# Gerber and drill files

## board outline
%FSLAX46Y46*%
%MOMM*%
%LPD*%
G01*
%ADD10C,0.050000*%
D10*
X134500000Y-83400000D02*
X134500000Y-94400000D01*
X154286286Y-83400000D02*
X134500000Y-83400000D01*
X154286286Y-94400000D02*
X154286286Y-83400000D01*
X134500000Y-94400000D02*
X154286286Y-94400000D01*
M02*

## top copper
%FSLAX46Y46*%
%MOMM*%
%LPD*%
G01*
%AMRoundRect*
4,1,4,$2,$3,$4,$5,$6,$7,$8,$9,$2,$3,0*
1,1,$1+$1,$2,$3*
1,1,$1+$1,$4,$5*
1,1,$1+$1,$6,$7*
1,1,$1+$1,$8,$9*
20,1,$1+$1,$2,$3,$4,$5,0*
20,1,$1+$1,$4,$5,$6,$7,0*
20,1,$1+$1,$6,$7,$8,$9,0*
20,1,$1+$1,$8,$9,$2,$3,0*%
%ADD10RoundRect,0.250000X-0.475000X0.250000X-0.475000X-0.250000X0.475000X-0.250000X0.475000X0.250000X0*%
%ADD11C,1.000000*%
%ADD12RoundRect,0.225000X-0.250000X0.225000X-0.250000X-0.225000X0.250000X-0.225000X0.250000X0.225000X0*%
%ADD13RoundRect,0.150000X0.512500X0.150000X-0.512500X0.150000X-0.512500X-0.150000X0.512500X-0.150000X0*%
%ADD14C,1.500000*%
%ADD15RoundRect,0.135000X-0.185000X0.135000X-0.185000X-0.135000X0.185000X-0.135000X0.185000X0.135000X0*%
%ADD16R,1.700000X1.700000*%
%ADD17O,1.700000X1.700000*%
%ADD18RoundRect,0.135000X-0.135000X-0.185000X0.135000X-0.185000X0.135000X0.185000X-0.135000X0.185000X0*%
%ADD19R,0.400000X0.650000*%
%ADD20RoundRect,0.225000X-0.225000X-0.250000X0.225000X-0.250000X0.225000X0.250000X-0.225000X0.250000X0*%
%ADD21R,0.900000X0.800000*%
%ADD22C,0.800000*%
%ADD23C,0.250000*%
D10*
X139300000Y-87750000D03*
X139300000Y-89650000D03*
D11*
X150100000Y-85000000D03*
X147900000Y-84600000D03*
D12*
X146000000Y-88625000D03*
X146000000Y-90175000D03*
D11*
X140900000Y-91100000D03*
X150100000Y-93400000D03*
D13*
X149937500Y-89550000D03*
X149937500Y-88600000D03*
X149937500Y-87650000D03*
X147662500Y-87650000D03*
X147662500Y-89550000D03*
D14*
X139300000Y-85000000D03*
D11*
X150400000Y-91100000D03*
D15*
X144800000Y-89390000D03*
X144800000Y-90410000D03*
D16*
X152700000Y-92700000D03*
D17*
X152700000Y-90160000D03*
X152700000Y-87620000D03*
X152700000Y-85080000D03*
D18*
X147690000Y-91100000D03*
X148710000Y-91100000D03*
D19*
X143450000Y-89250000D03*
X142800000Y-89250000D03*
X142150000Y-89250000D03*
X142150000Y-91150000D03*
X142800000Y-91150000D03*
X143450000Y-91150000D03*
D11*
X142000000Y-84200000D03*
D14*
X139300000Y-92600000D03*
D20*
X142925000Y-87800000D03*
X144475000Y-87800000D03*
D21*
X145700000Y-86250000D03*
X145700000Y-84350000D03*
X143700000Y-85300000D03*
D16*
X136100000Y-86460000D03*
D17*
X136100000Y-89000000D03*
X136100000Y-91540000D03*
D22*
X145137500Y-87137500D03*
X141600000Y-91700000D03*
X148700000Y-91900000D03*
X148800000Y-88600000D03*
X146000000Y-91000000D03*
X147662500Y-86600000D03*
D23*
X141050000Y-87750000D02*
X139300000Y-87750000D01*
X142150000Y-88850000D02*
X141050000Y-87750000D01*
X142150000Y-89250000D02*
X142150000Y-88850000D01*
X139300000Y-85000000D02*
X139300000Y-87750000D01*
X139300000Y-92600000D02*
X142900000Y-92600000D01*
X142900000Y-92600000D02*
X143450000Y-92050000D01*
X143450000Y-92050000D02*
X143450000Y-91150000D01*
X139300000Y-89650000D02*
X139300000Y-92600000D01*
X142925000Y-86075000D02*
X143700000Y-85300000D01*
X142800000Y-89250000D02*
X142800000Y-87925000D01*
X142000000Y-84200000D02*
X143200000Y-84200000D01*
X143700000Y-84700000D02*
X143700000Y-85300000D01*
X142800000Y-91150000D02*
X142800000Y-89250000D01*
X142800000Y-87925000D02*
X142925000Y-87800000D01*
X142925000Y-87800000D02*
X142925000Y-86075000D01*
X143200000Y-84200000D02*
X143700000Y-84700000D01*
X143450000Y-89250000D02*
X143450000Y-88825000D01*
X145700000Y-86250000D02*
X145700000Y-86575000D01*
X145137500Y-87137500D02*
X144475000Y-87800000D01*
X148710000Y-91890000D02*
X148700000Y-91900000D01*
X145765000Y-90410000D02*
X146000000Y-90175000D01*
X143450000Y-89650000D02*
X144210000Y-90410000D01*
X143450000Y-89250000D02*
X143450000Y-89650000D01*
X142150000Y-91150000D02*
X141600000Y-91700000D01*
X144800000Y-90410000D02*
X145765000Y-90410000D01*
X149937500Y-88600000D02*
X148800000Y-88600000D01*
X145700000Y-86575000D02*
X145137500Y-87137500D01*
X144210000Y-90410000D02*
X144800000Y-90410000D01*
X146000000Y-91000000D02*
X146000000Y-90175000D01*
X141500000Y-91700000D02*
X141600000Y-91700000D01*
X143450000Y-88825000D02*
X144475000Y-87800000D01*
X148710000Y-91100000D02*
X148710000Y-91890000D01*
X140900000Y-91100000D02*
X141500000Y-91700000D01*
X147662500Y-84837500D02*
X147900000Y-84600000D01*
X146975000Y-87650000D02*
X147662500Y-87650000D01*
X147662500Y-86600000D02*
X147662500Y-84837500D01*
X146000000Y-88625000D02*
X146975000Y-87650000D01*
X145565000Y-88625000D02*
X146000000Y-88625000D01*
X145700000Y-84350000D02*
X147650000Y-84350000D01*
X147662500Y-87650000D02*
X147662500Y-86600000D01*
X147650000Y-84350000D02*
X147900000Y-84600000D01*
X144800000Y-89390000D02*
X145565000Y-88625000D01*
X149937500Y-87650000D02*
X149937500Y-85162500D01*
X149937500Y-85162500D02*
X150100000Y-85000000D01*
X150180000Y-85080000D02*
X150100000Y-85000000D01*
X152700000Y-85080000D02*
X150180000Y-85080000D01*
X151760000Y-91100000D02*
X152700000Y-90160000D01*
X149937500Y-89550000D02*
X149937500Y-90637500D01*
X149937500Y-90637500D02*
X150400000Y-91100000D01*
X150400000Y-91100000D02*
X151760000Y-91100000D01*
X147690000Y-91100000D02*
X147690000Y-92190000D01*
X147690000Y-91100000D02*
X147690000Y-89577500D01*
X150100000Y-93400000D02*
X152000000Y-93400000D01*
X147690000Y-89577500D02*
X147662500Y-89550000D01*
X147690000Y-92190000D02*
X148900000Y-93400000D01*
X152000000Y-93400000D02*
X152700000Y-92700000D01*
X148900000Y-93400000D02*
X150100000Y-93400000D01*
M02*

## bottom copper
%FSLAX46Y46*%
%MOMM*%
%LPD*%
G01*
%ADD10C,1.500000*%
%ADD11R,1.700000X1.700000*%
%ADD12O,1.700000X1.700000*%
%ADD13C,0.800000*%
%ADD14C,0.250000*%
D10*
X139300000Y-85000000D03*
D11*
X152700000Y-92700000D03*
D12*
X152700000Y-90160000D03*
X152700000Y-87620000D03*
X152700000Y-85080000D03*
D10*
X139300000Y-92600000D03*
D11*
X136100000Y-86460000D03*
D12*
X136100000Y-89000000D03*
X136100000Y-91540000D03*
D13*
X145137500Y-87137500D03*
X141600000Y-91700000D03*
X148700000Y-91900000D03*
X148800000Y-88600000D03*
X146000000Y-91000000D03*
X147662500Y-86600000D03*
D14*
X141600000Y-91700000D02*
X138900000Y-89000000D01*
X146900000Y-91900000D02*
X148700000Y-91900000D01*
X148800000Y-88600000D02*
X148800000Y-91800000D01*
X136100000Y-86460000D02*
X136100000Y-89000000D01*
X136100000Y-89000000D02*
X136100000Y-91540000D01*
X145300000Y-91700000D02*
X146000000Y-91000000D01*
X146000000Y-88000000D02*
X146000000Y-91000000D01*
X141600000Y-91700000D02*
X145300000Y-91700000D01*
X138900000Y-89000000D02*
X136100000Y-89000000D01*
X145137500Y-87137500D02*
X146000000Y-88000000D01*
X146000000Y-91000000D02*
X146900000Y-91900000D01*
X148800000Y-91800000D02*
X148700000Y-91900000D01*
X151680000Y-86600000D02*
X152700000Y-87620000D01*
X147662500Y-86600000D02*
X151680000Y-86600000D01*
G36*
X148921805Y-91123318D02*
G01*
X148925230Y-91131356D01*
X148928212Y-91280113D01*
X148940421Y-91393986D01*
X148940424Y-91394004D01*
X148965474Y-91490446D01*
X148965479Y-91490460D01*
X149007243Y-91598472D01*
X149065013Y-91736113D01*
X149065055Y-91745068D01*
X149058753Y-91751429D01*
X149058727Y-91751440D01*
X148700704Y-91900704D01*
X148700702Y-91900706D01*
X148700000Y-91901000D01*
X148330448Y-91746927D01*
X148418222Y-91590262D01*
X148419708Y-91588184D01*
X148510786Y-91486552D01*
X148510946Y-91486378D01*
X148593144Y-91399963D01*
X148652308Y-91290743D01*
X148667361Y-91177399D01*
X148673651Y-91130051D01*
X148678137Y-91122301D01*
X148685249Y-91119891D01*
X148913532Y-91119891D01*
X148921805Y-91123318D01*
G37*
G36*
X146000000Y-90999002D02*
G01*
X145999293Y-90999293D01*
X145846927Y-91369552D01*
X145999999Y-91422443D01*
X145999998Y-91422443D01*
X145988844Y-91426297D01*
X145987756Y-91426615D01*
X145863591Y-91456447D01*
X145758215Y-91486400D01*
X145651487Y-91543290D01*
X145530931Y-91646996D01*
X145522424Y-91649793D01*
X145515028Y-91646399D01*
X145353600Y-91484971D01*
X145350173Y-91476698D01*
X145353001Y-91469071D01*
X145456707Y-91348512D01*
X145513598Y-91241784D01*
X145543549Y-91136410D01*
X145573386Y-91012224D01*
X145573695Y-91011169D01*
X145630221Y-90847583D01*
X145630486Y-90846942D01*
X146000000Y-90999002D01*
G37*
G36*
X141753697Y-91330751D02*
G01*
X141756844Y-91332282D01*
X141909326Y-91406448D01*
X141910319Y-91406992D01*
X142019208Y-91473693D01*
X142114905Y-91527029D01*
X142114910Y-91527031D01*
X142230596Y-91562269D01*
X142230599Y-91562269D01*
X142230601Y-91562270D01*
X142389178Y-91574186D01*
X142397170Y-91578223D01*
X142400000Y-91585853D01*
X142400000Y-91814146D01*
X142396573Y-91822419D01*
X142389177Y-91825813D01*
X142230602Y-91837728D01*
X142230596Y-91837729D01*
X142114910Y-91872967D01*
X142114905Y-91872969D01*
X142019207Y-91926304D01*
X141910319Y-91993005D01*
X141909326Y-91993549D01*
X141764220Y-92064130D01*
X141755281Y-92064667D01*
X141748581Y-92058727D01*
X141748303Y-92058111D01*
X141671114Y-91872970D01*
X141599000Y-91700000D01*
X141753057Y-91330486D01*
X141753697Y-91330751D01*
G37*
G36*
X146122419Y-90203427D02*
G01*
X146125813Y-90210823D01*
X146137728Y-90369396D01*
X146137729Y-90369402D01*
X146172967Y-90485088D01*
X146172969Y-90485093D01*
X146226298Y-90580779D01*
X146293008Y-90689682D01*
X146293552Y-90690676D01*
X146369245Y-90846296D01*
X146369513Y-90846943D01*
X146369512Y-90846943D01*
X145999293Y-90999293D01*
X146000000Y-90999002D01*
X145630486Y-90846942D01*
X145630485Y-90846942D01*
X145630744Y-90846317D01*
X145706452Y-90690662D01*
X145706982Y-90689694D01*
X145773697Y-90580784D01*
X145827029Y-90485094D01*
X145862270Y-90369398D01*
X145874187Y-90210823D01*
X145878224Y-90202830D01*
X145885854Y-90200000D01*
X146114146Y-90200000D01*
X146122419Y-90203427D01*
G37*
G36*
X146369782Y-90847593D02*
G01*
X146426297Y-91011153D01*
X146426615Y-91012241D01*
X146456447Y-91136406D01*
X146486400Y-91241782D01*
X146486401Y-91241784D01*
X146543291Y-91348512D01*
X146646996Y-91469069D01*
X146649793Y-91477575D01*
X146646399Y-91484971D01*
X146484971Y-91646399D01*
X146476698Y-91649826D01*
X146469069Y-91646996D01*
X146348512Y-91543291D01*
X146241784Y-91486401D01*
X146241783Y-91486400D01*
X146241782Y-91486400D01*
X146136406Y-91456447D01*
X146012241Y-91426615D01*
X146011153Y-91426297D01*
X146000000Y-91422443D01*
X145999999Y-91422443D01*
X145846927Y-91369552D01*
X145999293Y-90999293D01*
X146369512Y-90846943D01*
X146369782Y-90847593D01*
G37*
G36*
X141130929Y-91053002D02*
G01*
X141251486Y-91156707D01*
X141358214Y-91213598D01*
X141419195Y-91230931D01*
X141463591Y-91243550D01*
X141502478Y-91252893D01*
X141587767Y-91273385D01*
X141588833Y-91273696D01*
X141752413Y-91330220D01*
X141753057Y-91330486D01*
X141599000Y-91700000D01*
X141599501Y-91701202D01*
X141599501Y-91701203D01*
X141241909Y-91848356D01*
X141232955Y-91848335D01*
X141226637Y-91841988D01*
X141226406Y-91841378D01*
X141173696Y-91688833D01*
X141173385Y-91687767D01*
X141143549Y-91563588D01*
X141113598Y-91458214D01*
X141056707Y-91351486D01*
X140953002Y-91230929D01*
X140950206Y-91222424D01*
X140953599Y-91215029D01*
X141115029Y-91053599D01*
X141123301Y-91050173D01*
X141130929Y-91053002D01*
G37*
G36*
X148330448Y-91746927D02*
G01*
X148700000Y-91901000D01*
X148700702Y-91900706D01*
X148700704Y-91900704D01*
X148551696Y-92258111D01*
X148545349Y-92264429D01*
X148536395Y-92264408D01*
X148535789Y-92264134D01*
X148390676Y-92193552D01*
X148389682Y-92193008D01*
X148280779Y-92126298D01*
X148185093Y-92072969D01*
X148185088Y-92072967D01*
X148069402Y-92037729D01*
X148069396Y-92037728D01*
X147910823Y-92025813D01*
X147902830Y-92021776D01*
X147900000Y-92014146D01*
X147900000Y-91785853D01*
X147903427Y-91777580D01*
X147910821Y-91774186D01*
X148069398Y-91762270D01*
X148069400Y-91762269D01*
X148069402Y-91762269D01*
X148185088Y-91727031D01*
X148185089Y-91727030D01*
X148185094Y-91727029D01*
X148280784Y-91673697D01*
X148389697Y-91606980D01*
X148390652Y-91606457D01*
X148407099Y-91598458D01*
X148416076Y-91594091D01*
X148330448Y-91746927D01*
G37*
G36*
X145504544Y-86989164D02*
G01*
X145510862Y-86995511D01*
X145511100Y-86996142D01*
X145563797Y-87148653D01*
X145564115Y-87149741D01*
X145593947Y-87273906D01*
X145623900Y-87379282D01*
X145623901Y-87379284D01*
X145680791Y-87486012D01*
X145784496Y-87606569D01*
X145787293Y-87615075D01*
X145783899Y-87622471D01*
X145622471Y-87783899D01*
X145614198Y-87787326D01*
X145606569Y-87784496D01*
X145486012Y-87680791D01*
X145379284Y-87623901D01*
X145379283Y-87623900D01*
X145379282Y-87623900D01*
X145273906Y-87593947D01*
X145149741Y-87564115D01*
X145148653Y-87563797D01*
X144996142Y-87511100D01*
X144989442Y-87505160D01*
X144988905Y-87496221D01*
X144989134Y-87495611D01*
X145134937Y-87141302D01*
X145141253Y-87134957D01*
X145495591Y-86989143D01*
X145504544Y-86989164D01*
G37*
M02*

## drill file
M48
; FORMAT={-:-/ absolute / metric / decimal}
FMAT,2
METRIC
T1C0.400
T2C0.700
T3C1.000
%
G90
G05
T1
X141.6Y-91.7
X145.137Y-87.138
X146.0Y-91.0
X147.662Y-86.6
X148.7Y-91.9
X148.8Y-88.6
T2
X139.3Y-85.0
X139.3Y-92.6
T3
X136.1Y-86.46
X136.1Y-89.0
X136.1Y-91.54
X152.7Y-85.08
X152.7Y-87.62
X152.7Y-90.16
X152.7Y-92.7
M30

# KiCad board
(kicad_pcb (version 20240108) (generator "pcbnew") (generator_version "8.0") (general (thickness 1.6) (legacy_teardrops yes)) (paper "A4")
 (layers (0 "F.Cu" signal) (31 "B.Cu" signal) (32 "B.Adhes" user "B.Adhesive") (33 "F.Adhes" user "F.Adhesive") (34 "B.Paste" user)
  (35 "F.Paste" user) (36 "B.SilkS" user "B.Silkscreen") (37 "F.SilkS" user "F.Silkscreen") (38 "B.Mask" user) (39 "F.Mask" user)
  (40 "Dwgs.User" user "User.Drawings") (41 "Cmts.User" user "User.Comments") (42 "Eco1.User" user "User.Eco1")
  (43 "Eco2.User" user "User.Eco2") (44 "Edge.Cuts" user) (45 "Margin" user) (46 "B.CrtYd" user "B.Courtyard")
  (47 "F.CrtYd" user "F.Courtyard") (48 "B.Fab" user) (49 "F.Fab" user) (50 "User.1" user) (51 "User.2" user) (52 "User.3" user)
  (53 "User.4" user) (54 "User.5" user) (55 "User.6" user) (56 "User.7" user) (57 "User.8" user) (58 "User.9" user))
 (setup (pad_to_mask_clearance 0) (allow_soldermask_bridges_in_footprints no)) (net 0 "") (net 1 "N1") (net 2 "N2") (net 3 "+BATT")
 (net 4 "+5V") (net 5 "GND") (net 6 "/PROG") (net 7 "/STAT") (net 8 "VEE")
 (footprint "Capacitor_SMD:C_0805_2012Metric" (layer "F.Cu") (at 139.3 88.7 -90)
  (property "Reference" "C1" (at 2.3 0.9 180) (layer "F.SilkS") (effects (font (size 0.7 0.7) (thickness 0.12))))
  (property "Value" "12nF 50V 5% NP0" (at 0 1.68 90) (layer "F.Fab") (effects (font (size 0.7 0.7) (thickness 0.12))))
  (pad "1" smd roundrect (at -0.95 0 270) (size 1 1.45) (layers "F.Cu" "F.Paste" "F.Mask") (roundrect_rratio 0.25) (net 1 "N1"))
  (pad "2" smd roundrect (at 0.95 0 270) (size 1 1.45) (layers "F.Cu" "F.Paste" "F.Mask") (roundrect_rratio 0.25) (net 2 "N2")))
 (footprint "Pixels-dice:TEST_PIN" (layer "F.Cu") (at 150.1 85)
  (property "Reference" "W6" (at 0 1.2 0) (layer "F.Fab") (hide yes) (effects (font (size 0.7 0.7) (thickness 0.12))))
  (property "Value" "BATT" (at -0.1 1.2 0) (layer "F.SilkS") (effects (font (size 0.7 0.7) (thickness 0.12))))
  (pad "1" smd circle (at 0 0) (size 1 1) (layers "F.Cu" "F.Mask") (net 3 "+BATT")))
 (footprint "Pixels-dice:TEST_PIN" (layer "F.Cu") (at 147.9 84.6)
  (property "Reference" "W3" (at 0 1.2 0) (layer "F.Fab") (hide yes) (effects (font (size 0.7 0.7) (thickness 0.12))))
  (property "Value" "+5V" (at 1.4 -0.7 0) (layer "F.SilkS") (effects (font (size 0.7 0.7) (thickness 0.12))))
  (pad "1" smd circle (at 0 0) (size 1 1) (layers "F.Cu" "F.Mask") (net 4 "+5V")))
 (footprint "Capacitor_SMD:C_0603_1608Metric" (layer "F.Cu") (at 146 89.4 -90)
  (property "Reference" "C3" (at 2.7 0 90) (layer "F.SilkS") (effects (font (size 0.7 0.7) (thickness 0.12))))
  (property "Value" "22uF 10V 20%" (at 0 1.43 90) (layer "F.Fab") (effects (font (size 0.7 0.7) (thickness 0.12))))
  (pad "1" smd roundrect (at -0.775 0 270) (size 0.9 0.95) (layers "F.Cu" "F.Paste" "F.Mask") (roundrect_rratio 0.25) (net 4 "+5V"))
  (pad "2" smd roundrect (at 0.775 0 270) (size 0.9 0.95) (layers "F.Cu" "F.Paste" "F.Mask") (roundrect_rratio 0.25) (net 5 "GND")))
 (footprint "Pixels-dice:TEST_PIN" (layer "F.Cu") (at 140.9 91.1)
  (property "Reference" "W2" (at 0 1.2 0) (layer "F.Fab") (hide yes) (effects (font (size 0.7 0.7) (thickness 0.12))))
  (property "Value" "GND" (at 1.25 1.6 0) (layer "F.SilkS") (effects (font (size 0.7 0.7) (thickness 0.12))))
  (pad "1" smd circle (at 0 0) (size 1 1) (layers "F.Cu" "F.Mask") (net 5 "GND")))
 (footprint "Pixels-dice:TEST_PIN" (layer "F.Cu") (at 150.1 93.4)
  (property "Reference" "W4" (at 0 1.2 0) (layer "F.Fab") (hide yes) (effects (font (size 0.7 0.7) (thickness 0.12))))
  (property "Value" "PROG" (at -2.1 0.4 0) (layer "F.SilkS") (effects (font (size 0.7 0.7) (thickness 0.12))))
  (pad "1" smd circle (at 0 0) (size 1 1) (layers "F.Cu" "F.Mask") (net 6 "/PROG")))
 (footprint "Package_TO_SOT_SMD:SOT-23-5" (layer "F.Cu") (at 148.8 88.6 180)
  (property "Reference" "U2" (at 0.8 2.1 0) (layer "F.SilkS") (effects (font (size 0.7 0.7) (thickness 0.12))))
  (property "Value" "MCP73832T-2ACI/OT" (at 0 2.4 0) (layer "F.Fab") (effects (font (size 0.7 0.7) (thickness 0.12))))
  (pad "1" smd roundrect (at -1.1375 -0.95 180) (size 1.325 0.6) (layers "F.Cu" "F.Paste" "F.Mask") (roundrect_rratio 0.25) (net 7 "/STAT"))
  (pad "2" smd roundrect (at -1.1375 0 180) (size 1.325 0.6) (layers "F.Cu" "F.Paste" "F.Mask") (roundrect_rratio 0.25) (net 5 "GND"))
  (pad "3" smd roundrect (at -1.1375 0.95 180) (size 1.325 0.6) (layers "F.Cu" "F.Paste" "F.Mask") (roundrect_rratio 0.25) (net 3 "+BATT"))
  (pad "4" smd roundrect (at 1.1375 0.95 180) (size 1.325 0.6) (layers "F.Cu" "F.Paste" "F.Mask") (roundrect_rratio 0.25) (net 4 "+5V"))
  (pad "5" smd roundrect (at 1.1375 -0.95 180) (size 1.325 0.6) (layers "F.Cu" "F.Paste" "F.Mask") (roundrect_rratio 0.25) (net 6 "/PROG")))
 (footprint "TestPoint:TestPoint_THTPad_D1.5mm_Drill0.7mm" (layer "F.Cu") (at 139.3 85)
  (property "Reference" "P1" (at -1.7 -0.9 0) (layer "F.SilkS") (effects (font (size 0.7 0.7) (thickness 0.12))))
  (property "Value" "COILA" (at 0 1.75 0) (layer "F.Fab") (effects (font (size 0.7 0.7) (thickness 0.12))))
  (pad "1" thru_hole circle (at 0 0) (size 1.5 1.5) (drill 0.7) (layers "*.Cu" "*.Mask") (remove_unused_layers no) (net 1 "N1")))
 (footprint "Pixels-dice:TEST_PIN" (layer "F.Cu") (at 150.4 91.1)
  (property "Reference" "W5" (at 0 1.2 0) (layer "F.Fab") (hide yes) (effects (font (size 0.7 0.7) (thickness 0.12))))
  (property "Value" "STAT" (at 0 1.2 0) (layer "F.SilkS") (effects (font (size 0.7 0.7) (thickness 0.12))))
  (pad "1" smd circle (at 0 0) (size 1 1) (layers "F.Cu" "F.Mask") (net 7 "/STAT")))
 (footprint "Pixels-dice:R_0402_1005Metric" (layer "F.Cu") (at 144.8 89.9 -90)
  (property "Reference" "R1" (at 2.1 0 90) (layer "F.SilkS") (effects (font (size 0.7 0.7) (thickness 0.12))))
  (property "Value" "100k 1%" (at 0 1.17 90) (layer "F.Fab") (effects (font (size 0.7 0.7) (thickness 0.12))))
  (pad "1" smd roundrect (at -0.51 0 270) (size 0.54 0.64) (layers "F.Cu" "F.Paste" "F.Mask") (roundrect_rratio 0.25) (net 4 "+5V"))
  (pad "2" smd roundrect (at 0.51 0 270) (size 0.54 0.64) (layers "F.Cu" "F.Paste" "F.Mask") (roundrect_rratio 0.25) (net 5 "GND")))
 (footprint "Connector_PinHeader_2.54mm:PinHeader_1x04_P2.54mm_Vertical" (layer "F.Cu") (at 152.7 92.7 180)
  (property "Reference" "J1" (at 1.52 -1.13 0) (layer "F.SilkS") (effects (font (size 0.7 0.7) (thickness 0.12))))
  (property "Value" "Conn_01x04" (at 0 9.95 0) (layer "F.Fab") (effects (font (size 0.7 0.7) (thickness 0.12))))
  (pad "1" thru_hole rect (at 0 0 180) (size 1.7 1.7) (drill 1) (layers "*.Cu" "*.Mask") (remove_unused_layers no) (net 6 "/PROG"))
  (pad "2" thru_hole oval (at 0 2.54 180) (size 1.7 1.7) (drill 1) (layers "*.Cu" "*.Mask") (remove_unused_layers no) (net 7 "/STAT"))
  (pad "3" thru_hole oval (at 0 5.08 180) (size 1.7 1.7) (drill 1) (layers "*.Cu" "*.Mask") (remove_unused_layers no) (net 4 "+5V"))
  (pad "4" thru_hole oval (at 0 7.62 180) (size 1.7 1.7) (drill 1) (layers "*.Cu" "*.Mask") (remove_unused_layers no) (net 3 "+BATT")))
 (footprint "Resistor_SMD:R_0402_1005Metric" (layer "F.Cu") (at 148.2 91.1)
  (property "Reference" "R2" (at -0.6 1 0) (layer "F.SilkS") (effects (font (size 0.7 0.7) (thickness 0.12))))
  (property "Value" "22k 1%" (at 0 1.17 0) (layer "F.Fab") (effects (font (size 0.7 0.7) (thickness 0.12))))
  (pad "1" smd roundrect (at -0.51 0) (size 0.54 0.64) (layers "F.Cu" "F.Paste" "F.Mask") (roundrect_rratio 0.25) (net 6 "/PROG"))
  (pad "2" smd roundrect (at 0.51 0) (size 0.54 0.64) (layers "F.Cu" "F.Paste" "F.Mask") (roundrect_rratio 0.25) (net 5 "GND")))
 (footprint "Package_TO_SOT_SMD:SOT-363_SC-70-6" (layer "F.Cu") (at 142.8 90.2 -90)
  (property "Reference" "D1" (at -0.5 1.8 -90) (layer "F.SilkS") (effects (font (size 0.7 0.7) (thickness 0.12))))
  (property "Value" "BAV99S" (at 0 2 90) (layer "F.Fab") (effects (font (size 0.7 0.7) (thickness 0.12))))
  (pad "1" smd rect (at -0.95 -0.65 270) (size 0.65 0.4) (layers "F.Cu" "F.Paste" "F.Mask") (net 5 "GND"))
  (pad "2" smd rect (at -0.95 0 270) (size 0.65 0.4) (layers "F.Cu" "F.Paste" "F.Mask") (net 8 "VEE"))
  (pad "3" smd rect (at -0.95 0.65 270) (size 0.65 0.4) (layers "F.Cu" "F.Paste" "F.Mask") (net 1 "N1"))
  (pad "4" smd rect (at 0.95 0.65 270) (size 0.65 0.4) (layers "F.Cu" "F.Paste" "F.Mask") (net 5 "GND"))
  (pad "5" smd rect (at 0.95 0 270) (size 0.65 0.4) (layers "F.Cu" "F.Paste" "F.Mask") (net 8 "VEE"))
  (pad "6" smd rect (at 0.95 -0.65 270) (size 0.65 0.4) (layers "F.Cu" "F.Paste" "F.Mask") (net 2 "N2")))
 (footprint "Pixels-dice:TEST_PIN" (layer "F.Cu") (at 142 84.2)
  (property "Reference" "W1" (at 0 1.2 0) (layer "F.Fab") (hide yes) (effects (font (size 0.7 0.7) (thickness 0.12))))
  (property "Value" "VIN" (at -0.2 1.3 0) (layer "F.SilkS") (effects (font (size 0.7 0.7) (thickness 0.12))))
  (pad "1" smd circle (at 0 0) (size 1 1) (layers "F.Cu" "F.Mask") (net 8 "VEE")))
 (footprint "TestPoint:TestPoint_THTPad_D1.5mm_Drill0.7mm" (layer "F.Cu") (at 139.3 92.6)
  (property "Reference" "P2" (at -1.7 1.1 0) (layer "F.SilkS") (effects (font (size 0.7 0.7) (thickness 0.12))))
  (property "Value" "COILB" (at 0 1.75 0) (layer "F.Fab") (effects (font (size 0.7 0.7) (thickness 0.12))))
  (pad "1" thru_hole circle (at 0 0) (size 1.5 1.5) (drill 0.7) (layers "*.Cu" "*.Mask") (remove_unused_layers no) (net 2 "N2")))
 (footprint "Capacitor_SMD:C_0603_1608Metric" (layer "F.Cu") (at 143.7 87.8)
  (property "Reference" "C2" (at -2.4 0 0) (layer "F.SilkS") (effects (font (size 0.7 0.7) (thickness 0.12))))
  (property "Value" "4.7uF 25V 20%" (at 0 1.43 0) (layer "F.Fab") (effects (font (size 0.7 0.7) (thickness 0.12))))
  (pad "1" smd roundrect (at -0.775 0) (size 0.9 0.95) (layers "F.Cu" "F.Paste" "F.Mask") (roundrect_rratio 0.25) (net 8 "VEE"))
  (pad "2" smd roundrect (at 0.775 0) (size 0.9 0.95) (layers "F.Cu" "F.Paste" "F.Mask") (roundrect_rratio 0.25) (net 5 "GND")))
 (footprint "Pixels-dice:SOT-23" (layer "F.Cu") (at 144.7 85.3)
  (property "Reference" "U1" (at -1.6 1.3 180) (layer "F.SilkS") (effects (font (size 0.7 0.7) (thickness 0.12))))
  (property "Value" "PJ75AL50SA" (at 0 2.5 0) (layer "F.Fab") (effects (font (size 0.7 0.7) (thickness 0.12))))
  (pad "1" smd rect (at 1 0.95 180) (size 0.9 0.8) (layers "F.Cu" "F.Paste" "F.Mask") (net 5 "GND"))
  (pad "2" smd rect (at 1 -0.95 180) (size 0.9 0.8) (layers "F.Cu" "F.Paste" "F.Mask") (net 4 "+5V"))
  (pad "3" smd rect (at -1 0 180) (size 0.9 0.8) (layers "F.Cu" "F.Paste" "F.Mask") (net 8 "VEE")))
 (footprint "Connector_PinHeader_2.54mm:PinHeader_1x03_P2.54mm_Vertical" (layer "F.Cu") (at 136.1 86.46)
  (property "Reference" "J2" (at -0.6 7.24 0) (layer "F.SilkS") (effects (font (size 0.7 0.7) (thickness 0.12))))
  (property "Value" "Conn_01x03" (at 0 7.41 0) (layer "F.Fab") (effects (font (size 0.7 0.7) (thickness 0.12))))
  (pad "1" thru_hole rect (at 0 0) (size 1.7 1.7) (drill 1) (layers "*.Cu" "*.Mask") (remove_unused_layers no) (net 5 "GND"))
  (pad "2" thru_hole oval (at 0 2.54) (size 1.7 1.7) (drill 1) (layers "*.Cu" "*.Mask") (remove_unused_layers no) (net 5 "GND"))
  (pad "3" thru_hole oval (at 0 5.08) (size 1.7 1.7) (drill 1) (layers "*.Cu" "*.Mask") (remove_unused_layers no) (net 5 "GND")))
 (gr_line (start 134.5 83.4) (end 134.5 94.4) (stroke (width 0.05) (type solid)) (layer "Edge.Cuts"))
 (gr_line (start 154.286286 83.4) (end 134.5 83.4) (stroke (width 0.05) (type solid)) (layer "Edge.Cuts"))
 (gr_line (start 154.286286 94.4) (end 154.286286 83.4) (stroke (width 0.05) (type solid)) (layer "Edge.Cuts"))
 (gr_line (start 134.5 94.4) (end 154.286286 94.4) (stroke (width 0.05) (type solid)) (layer "Edge.Cuts"))
 (segment (start 141.05 87.75) (end 139.3 87.75) (width 0.25) (layer "F.Cu") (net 1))
 (segment (start 142.15 88.85) (end 141.05 87.75) (width 0.25) (layer "F.Cu") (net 1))
 (segment (start 142.15 89.25) (end 142.15 88.85) (width 0.25) (layer "F.Cu") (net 1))
 (segment (start 139.3 85) (end 139.3 87.75) (width 0.25) (layer "F.Cu") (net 1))
 (segment (start 139.3 92.6) (end 142.9 92.6) (width 0.25) (layer "F.Cu") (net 2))
 (segment (start 142.9 92.6) (end 143.45 92.05) (width 0.25) (layer "F.Cu") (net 2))
 (segment (start 143.45 92.05) (end 143.45 91.15) (width 0.25) (layer "F.Cu") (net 2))
 (segment (start 139.3 89.65) (end 139.3 92.6) (width 0.25) (layer "F.Cu") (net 2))
 (segment (start 142.925 86.075) (end 143.7 85.3) (width 0.25) (layer "F.Cu") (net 8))
 (segment (start 142.8 89.25) (end 142.8 87.925) (width 0.25) (layer "F.Cu") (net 8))
 (segment (start 142 84.2) (end 143.2 84.2) (width 0.25) (layer "F.Cu") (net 8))
 (segment (start 143.7 84.7) (end 143.7 85.3) (width 0.25) (layer "F.Cu") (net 8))
 (segment (start 142.8 91.15) (end 142.8 89.25) (width 0.25) (layer "F.Cu") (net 8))
 (segment (start 142.8 87.925) (end 142.925 87.8) (width 0.25) (layer "F.Cu") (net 8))
 (segment (start 142.925 87.8) (end 142.925 86.075) (width 0.25) (layer "F.Cu") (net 8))
 (segment (start 143.2 84.2) (end 143.7 84.7) (width 0.25) (layer "F.Cu") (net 8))
 (segment (start 143.45 89.25) (end 143.45 88.825) (width 0.25) (layer "F.Cu") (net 5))
 (segment (start 145.7 86.25) (end 145.7 86.575) (width 0.25) (layer "F.Cu") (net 5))
 (segment (start 145.1375 87.1375) (end 144.475 87.8) (width 0.25) (layer "F.Cu") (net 5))
 (segment (start 148.71 91.89) (end 148.7 91.9) (width 0.25) (layer "F.Cu") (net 5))
 (segment (start 145.765 90.41) (end 146 90.175) (width 0.25) (layer "F.Cu") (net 5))
 (segment (start 143.45 89.65) (end 144.21 90.41) (width 0.25) (layer "F.Cu") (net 5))
 (segment (start 143.45 89.25) (end 143.45 89.65) (width 0.25) (layer "F.Cu") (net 5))
 (segment (start 142.15 91.15) (end 141.6 91.7) (width 0.25) (layer "F.Cu") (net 5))
 (segment (start 144.8 90.41) (end 145.765 90.41) (width 0.25) (layer "F.Cu") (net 5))
 (segment (start 149.9375 88.6) (end 148.8 88.6) (width 0.25) (layer "F.Cu") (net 5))
 (segment (start 145.7 86.575) (end 145.1375 87.1375) (width 0.25) (layer "F.Cu") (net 5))
 (segment (start 144.21 90.41) (end 144.8 90.41) (width 0.25) (layer "F.Cu") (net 5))
 (segment (start 146 91) (end 146 90.175) (width 0.25) (layer "F.Cu") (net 5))
 (segment (start 141.5 91.7) (end 141.6 91.7) (width 0.25) (layer "F.Cu") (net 5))
 (segment (start 143.45 88.825) (end 144.475 87.8) (width 0.25) (layer "F.Cu") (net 5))
 (segment (start 148.71 91.1) (end 148.71 91.89) (width 0.25) (layer "F.Cu") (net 5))
 (segment (start 140.9 91.1) (end 141.5 91.7) (width 0.25) (layer "F.Cu") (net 5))
 (via (at 145.1375 87.1375) (size 0.8) (drill 0.4) (layers "F.Cu" "B.Cu") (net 5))
 (via (at 141.6 91.7) (size 0.8) (drill 0.4) (layers "F.Cu" "B.Cu") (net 5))
 (via (at 148.7 91.9) (size 0.8) (drill 0.4) (layers "F.Cu" "B.Cu") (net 5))
 (via (at 148.8 88.6) (size 0.8) (drill 0.4) (layers "F.Cu" "B.Cu") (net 5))
 (via (at 146 91) (size 0.8) (drill 0.4) (layers "F.Cu" "B.Cu") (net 5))
 (segment (start 141.6 91.7) (end 138.9 89) (width 0.25) (layer "B.Cu") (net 5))
 (segment (start 146.9 91.9) (end 148.7 91.9) (width 0.25) (layer "B.Cu") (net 5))
 (segment (start 148.8 88.6) (end 148.8 91.8) (width 0.25) (layer "B.Cu") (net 5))
 (segment (start 136.1 86.46) (end 136.1 89) (width 0.25) (layer "B.Cu") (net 5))
 (segment (start 136.1 89) (end 136.1 91.54) (width 0.25) (layer "B.Cu") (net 5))
 (segment (start 145.3 91.7) (end 146 91) (width 0.25) (layer "B.Cu") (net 5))
 (segment (start 146 88) (end 146 91) (width 0.25) (layer "B.Cu") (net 5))
 (segment (start 141.6 91.7) (end 145.3 91.7) (width 0.25) (layer "B.Cu") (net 5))
 (segment (start 138.9 89) (end 136.1 89) (width 0.25) (layer "B.Cu") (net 5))
 (segment (start 145.1375 87.1375) (end 146 88) (width 0.25) (layer "B.Cu") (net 5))
 (segment (start 146 91) (end 146.9 91.9) (width 0.25) (layer "B.Cu") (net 5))
 (segment (start 148.8 91.8) (end 148.7 91.9) (width 0.25) (layer "B.Cu") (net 5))
 (segment (start 147.6625 84.8375) (end 147.9 84.6) (width 0.25) (layer "F.Cu") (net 4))
 (segment (start 146.975 87.65) (end 147.6625 87.65) (width 0.25) (layer "F.Cu") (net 4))
 (segment (start 147.6625 86.6) (end 147.6625 84.8375) (width 0.25) (layer "F.Cu") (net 4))
 (segment (start 146 88.625) (end 146.975 87.65) (width 0.25) (layer "F.Cu") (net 4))
 (segment (start 145.565 88.625) (end 146 88.625) (width 0.25) (layer "F.Cu") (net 4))
 (segment (start 145.7 84.35) (end 147.65 84.35) (width 0.25) (layer "F.Cu") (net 4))
 (segment (start 147.6625 87.65) (end 147.6625 86.6) (width 0.25) (layer "F.Cu") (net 4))
 (segment (start 147.65 84.35) (end 147.9 84.6) (width 0.25) (layer "F.Cu") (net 4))
 (segment (start 144.8 89.39) (end 145.565 88.625) (width 0.25) (layer "F.Cu") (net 4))
 (via (at 147.6625 86.6) (size 0.8) (drill 0.4) (layers "F.Cu" "B.Cu") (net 4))
 (segment (start 151.68 86.6) (end 152.7 87.62) (width 0.25) (layer "B.Cu") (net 4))
 (segment (start 147.6625 86.6) (end 151.68 86.6) (width 0.25) (layer "B.Cu") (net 4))
 (segment (start 149.9375 87.65) (end 149.9375 85.1625) (width 0.25) (layer "F.Cu") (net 3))
 (segment (start 149.9375 85.1625) (end 150.1 85) (width 0.25) (layer "F.Cu") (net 3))
 (segment (start 150.18 85.08) (end 150.1 85) (width 0.25) (layer "F.Cu") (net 3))
 (segment (start 152.7 85.08) (end 150.18 85.08) (width 0.25) (layer "F.Cu") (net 3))
 (segment (start 151.76 91.1) (end 152.7 90.16) (width 0.25) (layer "F.Cu") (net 7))
 (segment (start 149.9375 89.55) (end 149.9375 90.6375) (width 0.25) (layer "F.Cu") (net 7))
 (segment (start 149.9375 90.6375) (end 150.4 91.1) (width 0.25) (layer "F.Cu") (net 7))
 (segment (start 150.4 91.1) (end 151.76 91.1) (width 0.25) (layer "F.Cu") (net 7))
 (segment (start 147.69 91.1) (end 147.69 92.19) (width 0.25) (layer "F.Cu") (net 6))
 (segment (start 147.69 91.1) (end 147.69 89.5775) (width 0.25) (layer "F.Cu") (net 6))
 (segment (start 150.1 93.4) (end 152 93.4) (width 0.25) (layer "F.Cu") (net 6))
 (segment (start 147.69 89.5775) (end 147.6625 89.55) (width 0.25) (layer "F.Cu") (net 6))
 (segment (start 147.69 92.19) (end 148.9 93.4) (width 0.25) (layer "F.Cu") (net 6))
 (segment (start 152 93.4) (end 152.7 92.7) (width 0.25) (layer "F.Cu") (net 6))
 (segment (start 148.9 93.4) (end 150.1 93.4) (width 0.25) (layer "F.Cu") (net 6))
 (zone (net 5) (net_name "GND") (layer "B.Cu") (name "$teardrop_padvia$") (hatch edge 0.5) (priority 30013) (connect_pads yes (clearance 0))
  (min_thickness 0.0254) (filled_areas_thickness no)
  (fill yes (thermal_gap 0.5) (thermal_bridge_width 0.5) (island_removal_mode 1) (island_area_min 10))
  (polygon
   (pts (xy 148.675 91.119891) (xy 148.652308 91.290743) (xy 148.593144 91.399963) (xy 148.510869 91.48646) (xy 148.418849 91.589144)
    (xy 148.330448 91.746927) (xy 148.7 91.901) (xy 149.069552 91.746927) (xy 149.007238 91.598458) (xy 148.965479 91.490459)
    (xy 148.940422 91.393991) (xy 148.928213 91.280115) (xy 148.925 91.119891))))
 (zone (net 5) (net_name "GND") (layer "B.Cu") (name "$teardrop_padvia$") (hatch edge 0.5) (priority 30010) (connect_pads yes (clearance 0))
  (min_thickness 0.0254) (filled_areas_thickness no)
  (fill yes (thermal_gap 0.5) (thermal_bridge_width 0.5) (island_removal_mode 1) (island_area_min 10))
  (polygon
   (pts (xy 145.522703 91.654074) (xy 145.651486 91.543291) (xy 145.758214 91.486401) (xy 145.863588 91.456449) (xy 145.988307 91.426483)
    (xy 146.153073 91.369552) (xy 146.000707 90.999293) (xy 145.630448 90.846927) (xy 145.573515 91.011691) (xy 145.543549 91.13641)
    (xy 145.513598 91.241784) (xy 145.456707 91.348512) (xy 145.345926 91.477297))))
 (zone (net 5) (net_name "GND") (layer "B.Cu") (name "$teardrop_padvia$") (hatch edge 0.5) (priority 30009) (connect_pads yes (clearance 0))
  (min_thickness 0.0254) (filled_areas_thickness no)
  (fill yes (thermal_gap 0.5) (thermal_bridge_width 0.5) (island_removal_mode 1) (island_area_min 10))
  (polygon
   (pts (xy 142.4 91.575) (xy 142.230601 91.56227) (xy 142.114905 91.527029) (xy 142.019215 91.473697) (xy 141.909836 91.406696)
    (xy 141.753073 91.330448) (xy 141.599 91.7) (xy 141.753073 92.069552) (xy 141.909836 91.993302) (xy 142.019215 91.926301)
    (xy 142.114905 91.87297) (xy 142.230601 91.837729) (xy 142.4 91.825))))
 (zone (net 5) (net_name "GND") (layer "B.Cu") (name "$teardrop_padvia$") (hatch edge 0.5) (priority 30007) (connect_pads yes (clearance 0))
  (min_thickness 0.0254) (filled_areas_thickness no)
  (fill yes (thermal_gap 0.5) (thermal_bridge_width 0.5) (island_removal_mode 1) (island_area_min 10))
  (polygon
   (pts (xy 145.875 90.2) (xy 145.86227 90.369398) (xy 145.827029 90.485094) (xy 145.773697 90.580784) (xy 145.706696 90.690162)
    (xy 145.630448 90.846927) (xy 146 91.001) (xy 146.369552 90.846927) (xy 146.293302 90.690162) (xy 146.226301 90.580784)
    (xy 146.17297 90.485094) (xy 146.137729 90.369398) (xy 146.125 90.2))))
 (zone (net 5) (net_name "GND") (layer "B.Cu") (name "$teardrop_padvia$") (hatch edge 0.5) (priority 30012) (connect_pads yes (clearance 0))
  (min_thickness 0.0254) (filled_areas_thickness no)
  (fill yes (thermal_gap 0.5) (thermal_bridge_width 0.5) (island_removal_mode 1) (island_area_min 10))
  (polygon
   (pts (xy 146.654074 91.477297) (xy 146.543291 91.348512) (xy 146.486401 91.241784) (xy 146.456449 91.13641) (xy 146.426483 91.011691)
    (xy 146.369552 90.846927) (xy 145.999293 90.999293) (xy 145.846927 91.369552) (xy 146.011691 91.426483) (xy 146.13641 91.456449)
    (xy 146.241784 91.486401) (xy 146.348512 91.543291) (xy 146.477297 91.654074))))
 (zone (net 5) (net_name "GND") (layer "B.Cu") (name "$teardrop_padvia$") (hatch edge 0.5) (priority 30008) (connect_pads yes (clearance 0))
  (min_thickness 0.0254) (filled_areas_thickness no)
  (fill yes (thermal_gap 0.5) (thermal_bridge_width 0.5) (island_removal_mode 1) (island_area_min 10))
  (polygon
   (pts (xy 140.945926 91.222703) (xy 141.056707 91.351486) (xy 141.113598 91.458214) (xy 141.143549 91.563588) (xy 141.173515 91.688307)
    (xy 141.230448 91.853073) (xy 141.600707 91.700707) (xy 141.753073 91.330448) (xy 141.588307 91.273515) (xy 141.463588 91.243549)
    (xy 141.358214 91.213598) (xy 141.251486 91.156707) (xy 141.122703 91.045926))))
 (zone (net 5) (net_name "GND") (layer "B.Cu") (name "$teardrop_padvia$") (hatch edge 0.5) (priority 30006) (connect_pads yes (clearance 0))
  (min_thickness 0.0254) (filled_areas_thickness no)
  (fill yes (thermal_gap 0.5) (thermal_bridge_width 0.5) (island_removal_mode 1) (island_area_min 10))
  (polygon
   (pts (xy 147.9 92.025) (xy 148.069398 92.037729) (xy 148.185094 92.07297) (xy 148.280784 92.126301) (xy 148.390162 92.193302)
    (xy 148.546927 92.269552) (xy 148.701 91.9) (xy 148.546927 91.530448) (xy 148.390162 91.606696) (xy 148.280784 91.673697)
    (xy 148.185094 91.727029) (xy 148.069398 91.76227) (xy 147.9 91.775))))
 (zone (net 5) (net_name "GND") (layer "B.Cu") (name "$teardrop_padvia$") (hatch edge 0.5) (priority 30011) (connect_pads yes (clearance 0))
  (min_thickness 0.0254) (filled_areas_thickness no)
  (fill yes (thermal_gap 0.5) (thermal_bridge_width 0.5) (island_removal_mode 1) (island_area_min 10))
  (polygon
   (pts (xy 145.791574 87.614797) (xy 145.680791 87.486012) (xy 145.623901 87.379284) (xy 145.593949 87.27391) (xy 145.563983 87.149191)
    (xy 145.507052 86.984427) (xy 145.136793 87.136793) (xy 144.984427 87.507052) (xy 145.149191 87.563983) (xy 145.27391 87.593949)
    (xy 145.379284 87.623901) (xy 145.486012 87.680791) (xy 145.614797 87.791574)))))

